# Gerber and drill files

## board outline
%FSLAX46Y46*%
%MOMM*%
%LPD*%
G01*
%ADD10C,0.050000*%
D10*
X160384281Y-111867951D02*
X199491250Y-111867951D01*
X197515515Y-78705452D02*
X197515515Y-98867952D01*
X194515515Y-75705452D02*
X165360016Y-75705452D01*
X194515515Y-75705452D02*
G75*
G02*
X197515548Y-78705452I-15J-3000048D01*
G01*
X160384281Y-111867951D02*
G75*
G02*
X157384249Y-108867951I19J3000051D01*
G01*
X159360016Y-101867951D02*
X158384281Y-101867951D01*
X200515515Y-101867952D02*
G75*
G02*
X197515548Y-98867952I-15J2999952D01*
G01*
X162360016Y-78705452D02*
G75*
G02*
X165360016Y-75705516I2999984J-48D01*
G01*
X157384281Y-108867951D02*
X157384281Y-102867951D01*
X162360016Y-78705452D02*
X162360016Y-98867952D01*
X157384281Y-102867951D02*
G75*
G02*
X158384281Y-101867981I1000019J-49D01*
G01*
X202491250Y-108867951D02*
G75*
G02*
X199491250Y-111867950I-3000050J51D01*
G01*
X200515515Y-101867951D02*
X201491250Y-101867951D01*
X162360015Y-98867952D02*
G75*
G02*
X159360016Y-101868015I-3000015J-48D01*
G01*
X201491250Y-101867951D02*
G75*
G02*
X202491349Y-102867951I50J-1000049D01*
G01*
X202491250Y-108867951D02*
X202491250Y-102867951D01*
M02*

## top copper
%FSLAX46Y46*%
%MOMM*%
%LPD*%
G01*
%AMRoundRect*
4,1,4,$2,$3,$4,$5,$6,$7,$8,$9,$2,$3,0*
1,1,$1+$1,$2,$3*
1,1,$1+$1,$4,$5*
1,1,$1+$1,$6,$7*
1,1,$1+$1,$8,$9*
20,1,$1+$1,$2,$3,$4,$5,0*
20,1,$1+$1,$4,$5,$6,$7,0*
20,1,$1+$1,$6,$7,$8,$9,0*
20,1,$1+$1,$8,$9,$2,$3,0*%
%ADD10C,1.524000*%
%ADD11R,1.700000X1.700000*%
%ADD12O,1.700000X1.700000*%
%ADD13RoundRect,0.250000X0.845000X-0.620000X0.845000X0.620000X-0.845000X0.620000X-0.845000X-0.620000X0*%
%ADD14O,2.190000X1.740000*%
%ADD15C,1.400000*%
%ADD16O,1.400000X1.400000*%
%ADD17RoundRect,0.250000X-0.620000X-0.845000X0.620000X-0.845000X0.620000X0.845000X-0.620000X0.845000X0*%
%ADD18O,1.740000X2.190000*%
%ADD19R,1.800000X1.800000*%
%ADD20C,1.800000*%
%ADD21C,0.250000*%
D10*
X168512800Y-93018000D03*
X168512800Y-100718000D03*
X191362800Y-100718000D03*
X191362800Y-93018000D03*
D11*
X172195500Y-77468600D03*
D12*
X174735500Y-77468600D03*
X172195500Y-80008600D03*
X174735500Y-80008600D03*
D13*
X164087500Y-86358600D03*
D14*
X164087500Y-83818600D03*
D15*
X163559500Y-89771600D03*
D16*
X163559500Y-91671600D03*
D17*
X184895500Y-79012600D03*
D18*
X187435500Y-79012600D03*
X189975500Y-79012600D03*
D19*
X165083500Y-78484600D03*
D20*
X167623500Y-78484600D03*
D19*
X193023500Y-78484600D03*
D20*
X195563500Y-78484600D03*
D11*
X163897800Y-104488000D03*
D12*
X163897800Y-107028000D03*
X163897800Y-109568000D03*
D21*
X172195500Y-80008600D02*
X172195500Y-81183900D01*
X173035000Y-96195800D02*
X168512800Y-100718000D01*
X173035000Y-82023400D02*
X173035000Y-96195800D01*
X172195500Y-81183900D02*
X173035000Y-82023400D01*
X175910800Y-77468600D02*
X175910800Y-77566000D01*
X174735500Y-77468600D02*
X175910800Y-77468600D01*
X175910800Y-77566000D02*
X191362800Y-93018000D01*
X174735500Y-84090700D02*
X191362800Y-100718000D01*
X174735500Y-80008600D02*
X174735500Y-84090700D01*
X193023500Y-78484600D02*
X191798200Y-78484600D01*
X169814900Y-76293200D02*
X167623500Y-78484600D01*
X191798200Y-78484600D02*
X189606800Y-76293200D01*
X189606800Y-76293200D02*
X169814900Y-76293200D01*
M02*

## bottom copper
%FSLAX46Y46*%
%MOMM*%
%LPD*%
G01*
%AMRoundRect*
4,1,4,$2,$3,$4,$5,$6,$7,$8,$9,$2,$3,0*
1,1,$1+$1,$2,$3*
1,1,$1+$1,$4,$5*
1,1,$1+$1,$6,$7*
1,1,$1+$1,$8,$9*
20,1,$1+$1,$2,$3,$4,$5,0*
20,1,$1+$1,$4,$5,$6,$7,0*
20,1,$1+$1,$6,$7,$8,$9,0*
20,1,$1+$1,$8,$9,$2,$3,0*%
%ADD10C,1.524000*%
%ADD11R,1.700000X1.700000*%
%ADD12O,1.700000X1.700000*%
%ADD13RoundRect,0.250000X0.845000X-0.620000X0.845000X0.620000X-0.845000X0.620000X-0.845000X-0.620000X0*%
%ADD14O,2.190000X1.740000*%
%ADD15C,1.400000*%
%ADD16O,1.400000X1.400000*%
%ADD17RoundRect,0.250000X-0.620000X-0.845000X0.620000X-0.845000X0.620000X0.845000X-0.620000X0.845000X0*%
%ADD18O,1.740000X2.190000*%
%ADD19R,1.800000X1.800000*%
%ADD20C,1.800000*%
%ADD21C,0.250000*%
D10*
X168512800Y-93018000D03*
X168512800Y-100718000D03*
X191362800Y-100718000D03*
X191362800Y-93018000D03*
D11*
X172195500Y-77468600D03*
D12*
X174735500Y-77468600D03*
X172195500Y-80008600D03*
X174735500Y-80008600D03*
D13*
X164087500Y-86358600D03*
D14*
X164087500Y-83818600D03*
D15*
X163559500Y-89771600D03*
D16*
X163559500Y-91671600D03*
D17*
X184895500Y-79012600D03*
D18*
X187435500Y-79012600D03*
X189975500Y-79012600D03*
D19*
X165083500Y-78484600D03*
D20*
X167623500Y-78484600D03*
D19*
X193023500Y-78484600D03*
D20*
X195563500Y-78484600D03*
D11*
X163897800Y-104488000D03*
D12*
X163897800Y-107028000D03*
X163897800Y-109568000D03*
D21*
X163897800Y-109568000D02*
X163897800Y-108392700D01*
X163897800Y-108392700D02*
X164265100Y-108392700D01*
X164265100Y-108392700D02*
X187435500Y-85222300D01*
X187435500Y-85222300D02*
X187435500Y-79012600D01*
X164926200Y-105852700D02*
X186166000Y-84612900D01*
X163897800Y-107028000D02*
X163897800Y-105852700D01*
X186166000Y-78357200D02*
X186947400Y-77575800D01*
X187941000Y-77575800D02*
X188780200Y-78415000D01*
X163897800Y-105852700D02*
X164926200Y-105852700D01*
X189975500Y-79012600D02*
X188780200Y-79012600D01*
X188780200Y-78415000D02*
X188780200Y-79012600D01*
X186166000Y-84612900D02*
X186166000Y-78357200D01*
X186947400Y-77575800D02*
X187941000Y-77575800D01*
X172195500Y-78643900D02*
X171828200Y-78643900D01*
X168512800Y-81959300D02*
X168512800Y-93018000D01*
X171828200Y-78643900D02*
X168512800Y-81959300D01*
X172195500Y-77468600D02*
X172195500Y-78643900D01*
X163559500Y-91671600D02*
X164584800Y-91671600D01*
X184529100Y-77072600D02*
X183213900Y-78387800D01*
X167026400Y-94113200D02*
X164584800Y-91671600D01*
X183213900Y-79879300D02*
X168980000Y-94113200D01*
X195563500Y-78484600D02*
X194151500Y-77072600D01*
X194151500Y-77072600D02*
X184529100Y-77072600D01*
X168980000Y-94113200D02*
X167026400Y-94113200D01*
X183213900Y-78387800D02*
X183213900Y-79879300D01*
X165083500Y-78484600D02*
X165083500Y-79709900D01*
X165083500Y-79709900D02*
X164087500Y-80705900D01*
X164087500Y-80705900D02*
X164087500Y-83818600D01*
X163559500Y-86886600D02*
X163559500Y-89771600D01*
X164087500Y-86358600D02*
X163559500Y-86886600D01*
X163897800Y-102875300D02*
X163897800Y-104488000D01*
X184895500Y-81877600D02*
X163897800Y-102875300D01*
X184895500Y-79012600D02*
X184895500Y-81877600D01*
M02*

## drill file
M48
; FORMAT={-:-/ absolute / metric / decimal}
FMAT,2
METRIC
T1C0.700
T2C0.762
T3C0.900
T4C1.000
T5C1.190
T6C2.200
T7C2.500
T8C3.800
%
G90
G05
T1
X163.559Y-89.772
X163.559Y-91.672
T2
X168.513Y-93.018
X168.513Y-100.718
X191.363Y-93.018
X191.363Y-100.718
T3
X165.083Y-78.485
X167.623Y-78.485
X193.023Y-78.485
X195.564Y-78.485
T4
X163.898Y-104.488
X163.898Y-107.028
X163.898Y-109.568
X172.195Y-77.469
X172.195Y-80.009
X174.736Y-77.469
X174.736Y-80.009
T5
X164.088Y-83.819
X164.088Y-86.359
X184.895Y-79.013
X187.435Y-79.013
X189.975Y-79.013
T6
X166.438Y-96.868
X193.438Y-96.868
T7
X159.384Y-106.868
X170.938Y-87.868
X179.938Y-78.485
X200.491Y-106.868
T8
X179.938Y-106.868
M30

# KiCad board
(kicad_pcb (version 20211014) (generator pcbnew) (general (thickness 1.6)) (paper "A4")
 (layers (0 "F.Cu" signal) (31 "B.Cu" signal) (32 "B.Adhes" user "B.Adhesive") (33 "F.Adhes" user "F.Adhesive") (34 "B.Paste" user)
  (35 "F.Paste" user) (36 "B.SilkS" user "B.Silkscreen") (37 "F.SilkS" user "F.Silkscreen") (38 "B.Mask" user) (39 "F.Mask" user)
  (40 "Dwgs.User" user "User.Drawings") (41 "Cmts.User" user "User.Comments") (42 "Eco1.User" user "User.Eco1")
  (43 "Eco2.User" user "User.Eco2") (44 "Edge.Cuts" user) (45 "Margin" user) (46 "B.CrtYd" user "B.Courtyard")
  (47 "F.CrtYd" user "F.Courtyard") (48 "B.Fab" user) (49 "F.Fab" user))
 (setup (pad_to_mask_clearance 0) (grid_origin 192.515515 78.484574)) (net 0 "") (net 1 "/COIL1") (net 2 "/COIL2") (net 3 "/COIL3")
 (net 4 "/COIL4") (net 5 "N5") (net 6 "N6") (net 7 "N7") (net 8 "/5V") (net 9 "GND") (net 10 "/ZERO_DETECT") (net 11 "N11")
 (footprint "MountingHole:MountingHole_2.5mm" (layer "F.Cu") (at 179.9378 78.4846)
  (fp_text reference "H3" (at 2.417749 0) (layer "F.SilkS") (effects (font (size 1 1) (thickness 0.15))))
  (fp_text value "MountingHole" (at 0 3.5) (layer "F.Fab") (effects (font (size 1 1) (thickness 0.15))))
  (pad "" np_thru_hole circle locked (at 0 0) (size 2.5 2.5) (drill 2.5) (layers *.Cu *.Mask)))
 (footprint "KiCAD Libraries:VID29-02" (layer "F.Cu") (at 180.1028 96.868)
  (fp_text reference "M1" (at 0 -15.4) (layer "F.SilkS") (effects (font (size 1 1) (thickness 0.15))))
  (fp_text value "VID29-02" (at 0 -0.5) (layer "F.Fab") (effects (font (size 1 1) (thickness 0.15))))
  (pad "" np_thru_hole circle locked (at -9.165 -9) (size 2.5 2.5) (drill 2.5) (layers *.Cu *.Mask))
  (pad "" np_thru_hole circle locked (at 13.335 0) (size 2.2 2.2) (drill 2.2) (layers *.Cu *.Mask))
  (pad "" np_thru_hole circle locked (at -0.165 10) (size 3.8 3.8) (drill 3.8) (layers *.Cu *.Mask))
  (pad "" np_thru_hole circle locked (at -13.665 0) (size 2.2 2.2) (drill 2.2) (layers *.Cu *.Mask))
  (pad "1" thru_hole circle locked (at -11.59 -3.85) (size 1.524 1.524) (drill 0.762) (layers *.Cu *.Mask) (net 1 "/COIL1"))
  (pad "2" thru_hole circle locked (at -11.59 3.85) (size 1.524 1.524) (drill 0.762) (layers *.Cu *.Mask) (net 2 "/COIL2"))
  (pad "3" thru_hole circle locked (at 11.26 3.85) (size 1.524 1.524) (drill 0.762) (layers *.Cu *.Mask) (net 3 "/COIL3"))
  (pad "4" thru_hole circle locked (at 11.26 -3.85) (size 1.524 1.524) (drill 0.762) (layers *.Cu *.Mask) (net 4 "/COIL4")))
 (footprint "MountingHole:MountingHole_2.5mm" (layer "F.Cu") (at 159.3843 106.868)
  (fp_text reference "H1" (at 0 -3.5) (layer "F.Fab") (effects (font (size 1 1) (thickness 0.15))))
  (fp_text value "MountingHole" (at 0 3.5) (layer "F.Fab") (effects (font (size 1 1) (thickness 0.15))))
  (pad "" np_thru_hole circle locked (at 0 0) (size 2.5 2.5) (drill 2.5) (layers *.Cu *.Mask)))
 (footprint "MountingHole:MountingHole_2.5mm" (layer "F.Cu") (at 200.4913 106.868)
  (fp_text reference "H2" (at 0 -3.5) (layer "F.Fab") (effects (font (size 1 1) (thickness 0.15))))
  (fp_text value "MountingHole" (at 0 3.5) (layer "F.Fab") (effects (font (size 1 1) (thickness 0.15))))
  (pad "" np_thru_hole circle locked (at 0 0) (size 2.5 2.5) (drill 2.5) (layers *.Cu *.Mask)))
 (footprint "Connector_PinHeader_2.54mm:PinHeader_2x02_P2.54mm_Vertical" (layer "F.Cu") (at 172.1955 77.4686)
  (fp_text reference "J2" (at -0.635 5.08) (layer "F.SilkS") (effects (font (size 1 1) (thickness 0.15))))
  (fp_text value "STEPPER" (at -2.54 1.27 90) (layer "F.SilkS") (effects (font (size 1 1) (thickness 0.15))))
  (pad "1" thru_hole rect locked (at 0 0) (size 1.7 1.7) (drill 1) (layers *.Cu *.Mask) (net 1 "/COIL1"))
  (pad "2" thru_hole oval locked (at 2.54 0) (size 1.7 1.7) (drill 1) (layers *.Cu *.Mask) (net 4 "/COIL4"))
  (pad "3" thru_hole oval locked (at 0 2.54) (size 1.7 1.7) (drill 1) (layers *.Cu *.Mask) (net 2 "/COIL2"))
  (pad "4" thru_hole oval locked (at 2.54 2.54) (size 1.7 1.7) (drill 1) (layers *.Cu *.Mask) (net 3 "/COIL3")))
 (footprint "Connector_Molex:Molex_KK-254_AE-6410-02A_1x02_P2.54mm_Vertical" (layer "F.Cu") (at 164.0875 86.3586 90)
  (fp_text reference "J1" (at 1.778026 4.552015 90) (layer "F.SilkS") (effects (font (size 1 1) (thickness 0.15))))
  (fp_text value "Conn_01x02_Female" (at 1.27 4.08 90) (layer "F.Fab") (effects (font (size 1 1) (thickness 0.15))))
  (pad "1" thru_hole roundrect (at 0 0 90) (size 1.74 2.19) (drill 1.19) (layers *.Cu *.Mask) (roundrect_rratio 0.143678) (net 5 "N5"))
  (pad "2" thru_hole oval (at 2.54 0 90) (size 1.74 2.19) (drill 1.19) (layers *.Cu *.Mask) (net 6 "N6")))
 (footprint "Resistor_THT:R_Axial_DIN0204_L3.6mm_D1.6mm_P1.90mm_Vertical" (layer "F.Cu") (at 163.5595 89.7716 -90)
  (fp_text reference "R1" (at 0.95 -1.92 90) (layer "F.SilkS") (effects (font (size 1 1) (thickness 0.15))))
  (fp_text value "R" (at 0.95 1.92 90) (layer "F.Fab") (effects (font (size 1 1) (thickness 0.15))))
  (pad "1" thru_hole circle (at 0 0 270) (size 1.4 1.4) (drill 0.7) (layers *.Cu *.Mask) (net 5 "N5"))
  (pad "2" thru_hole oval (at 1.9 0 270) (size 1.4 1.4) (drill 0.7) (layers *.Cu *.Mask) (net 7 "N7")))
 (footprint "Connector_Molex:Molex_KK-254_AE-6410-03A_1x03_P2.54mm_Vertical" (layer "F.Cu") (at 184.8955 79.0126)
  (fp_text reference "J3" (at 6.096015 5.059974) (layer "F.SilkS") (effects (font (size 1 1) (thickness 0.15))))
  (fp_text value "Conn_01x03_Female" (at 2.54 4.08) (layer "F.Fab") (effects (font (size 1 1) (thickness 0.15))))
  (pad "1" thru_hole roundrect (at 0 0) (size 1.74 2.19) (drill 1.19) (layers *.Cu *.Mask) (roundrect_rratio 0.143678) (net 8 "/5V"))
  (pad "2" thru_hole oval (at 2.54 0) (size 1.74 2.19) (drill 1.19) (layers *.Cu *.Mask) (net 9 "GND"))
  (pad "3" thru_hole oval (at 5.08 0) (size 1.74 2.19) (drill 1.19) (layers *.Cu *.Mask) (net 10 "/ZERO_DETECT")))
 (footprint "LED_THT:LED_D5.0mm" (layer "F.Cu") (at 165.0835 78.4846)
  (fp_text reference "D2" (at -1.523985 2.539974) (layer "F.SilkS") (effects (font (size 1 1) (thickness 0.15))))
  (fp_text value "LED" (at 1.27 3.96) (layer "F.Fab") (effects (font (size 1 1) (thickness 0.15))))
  (pad "1" thru_hole rect (at 0 0) (size 1.8 1.8) (drill 0.9) (layers *.Cu *.Mask) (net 6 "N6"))
  (pad "2" thru_hole circle (at 2.54 0) (size 1.8 1.8) (drill 0.9) (layers *.Cu *.Mask) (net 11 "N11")))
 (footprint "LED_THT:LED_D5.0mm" (layer "F.Cu") (at 193.0235 78.4846)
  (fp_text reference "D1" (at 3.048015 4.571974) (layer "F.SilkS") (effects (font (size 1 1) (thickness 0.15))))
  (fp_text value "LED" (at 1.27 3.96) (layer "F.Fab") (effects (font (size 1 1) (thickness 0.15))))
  (pad "1" thru_hole rect (at 0 0) (size 1.8 1.8) (drill 0.9) (layers *.Cu *.Mask) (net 11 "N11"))
  (pad "2" thru_hole circle (at 2.54 0) (size 1.8 1.8) (drill 0.9) (layers *.Cu *.Mask) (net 7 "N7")))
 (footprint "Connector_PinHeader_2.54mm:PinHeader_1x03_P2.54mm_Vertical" (layer "B.Cu") (at 163.8978 104.488 180)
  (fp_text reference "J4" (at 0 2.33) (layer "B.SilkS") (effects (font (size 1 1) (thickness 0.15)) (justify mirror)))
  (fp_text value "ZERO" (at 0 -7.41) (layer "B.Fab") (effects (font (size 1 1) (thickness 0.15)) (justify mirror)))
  (pad "1" thru_hole rect locked (at 0 0 180) (size 1.7 1.7) (drill 1) (layers *.Cu *.Mask) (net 8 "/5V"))
  (pad "2" thru_hole oval locked (at 0 -2.54 180) (size 1.7 1.7) (drill 1) (layers *.Cu *.Mask) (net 10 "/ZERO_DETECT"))
  (pad "3" thru_hole oval locked (at 0 -5.08 180) (size 1.7 1.7) (drill 1) (layers *.Cu *.Mask) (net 9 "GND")))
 (gr_line (start 160.384281 111.867951) (end 199.49125 111.867951) (layer "Edge.Cuts") (width 0.05))
 (gr_line (start 197.515515 78.705452) (end 197.515515 98.867952) (layer "Edge.Cuts") (width 0.05))
 (gr_line (start 194.515515 75.705452) (end 165.360016 75.705452) (layer "Edge.Cuts") (width 0.05))
 (gr_arc (start 194.515515 75.705452) (mid 196.636835 76.584132) (end 197.515515 78.705452) (layer "Edge.Cuts") (width 0.05))
 (gr_arc (start 160.384281 111.867951) (mid 158.262961 110.989271) (end 157.384281 108.867951) (layer "Edge.Cuts") (width 0.05))
 (gr_line (start 159.360016 101.867951) (end 158.384281 101.867951) (layer "Edge.Cuts") (width 0.05))
 (gr_arc (start 200.515515 101.867952) (mid 198.394195 100.989272) (end 197.515515 98.867952) (layer "Edge.Cuts") (width 0.05))
 (gr_arc (start 162.360016 78.705452) (mid 163.238696 76.584132) (end 165.360016 75.705452) (layer "Edge.Cuts") (width 0.05))
 (gr_line (start 157.384281 108.867951) (end 157.384281 102.867951) (layer "Edge.Cuts") (width 0.05))
 (gr_line (start 162.360016 78.705452) (end 162.360016 98.867952) (layer "Edge.Cuts") (width 0.05))
 (gr_arc (start 157.384281 102.867951) (mid 157.677174 102.160844) (end 158.384281 101.867951) (layer "Edge.Cuts") (width 0.05))
 (gr_arc (start 202.49125 108.867951) (mid 201.61257 110.989271) (end 199.49125 111.867951) (layer "Edge.Cuts") (width 0.05))
 (gr_line (start 200.515515 101.867951) (end 201.49125 101.867951) (layer "Edge.Cuts") (width 0.05))
 (gr_arc (start 162.360015 98.867952) (mid 161.481336 100.989272) (end 159.360016 101.867951) (layer "Edge.Cuts") (width 0.05))
 (gr_arc (start 201.49125 101.867951) (mid 202.198357 102.160844) (end 202.49125 102.867951) (layer "Edge.Cuts") (width 0.05))
 (gr_line (start 202.49125 108.867951) (end 202.49125 102.867951) (layer "Edge.Cuts") (width 0.05))
 (segment (start 163.8978 109.568) (end 163.8978 108.3927) (width 0.25) (layer "B.Cu") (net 9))
 (segment (start 163.8978 108.3927) (end 164.2651 108.3927) (width 0.25) (layer "B.Cu") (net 9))
 (segment (start 164.2651 108.3927) (end 187.4355 85.2223) (width 0.25) (layer "B.Cu") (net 9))
 (segment (start 187.4355 85.2223) (end 187.4355 79.0126) (width 0.25) (layer "B.Cu") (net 9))
 (segment (start 164.9262 105.8527) (end 186.166 84.6129) (width 0.25) (layer "B.Cu") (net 10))
 (segment (start 163.8978 107.028) (end 163.8978 105.8527) (width 0.25) (layer "B.Cu") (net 10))
 (segment (start 186.166 78.3572) (end 186.9474 77.5758) (width 0.25) (layer "B.Cu") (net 10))
 (segment (start 187.941 77.5758) (end 188.7802 78.415) (width 0.25) (layer "B.Cu") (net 10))
 (segment (start 163.8978 105.8527) (end 164.9262 105.8527) (width 0.25) (layer "B.Cu") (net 10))
 (segment (start 189.9755 79.0126) (end 188.7802 79.0126) (width 0.25) (layer "B.Cu") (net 10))
 (segment (start 188.7802 78.415) (end 188.7802 79.0126) (width 0.25) (layer "B.Cu") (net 10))
 (segment (start 186.166 84.6129) (end 186.166 78.3572) (width 0.25) (layer "B.Cu") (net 10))
 (segment (start 186.9474 77.5758) (end 187.941 77.5758) (width 0.25) (layer "B.Cu") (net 10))
 (segment (start 172.1955 80.0086) (end 172.1955 81.1839) (width 0.25) (layer "F.Cu") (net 2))
 (segment (start 173.035 96.1958) (end 168.5128 100.718) (width 0.25) (layer "F.Cu") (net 2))
 (segment (start 173.035 82.0234) (end 173.035 96.1958) (width 0.25) (layer "F.Cu") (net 2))
 (segment (start 172.1955 81.1839) (end 173.035 82.0234) (width 0.25) (layer "F.Cu") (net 2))
 (segment (start 172.1955 78.6439) (end 171.8282 78.6439) (width 0.25) (layer "B.Cu") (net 1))
 (segment (start 168.5128 81.9593) (end 168.5128 93.018) (width 0.25) (layer "B.Cu") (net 1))
 (segment (start 171.8282 78.6439) (end 168.5128 81.9593) (width 0.25) (layer "B.Cu") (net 1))
 (segment (start 172.1955 77.4686) (end 172.1955 78.6439) (width 0.25) (layer "B.Cu") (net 1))
 (segment (start 175.9108 77.4686) (end 175.9108 77.566) (width 0.25) (layer "F.Cu") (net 4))
 (segment (start 174.7355 77.4686) (end 175.9108 77.4686) (width 0.25) (layer "F.Cu") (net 4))
 (segment (start 175.9108 77.566) (end 191.3628 93.018) (width 0.25) (layer "F.Cu") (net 4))
 (segment (start 174.7355 84.0907) (end 191.3628 100.718) (width 0.25) (layer "F.Cu") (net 3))
 (segment (start 174.7355 80.0086) (end 174.7355 84.0907) (width 0.25) (layer "F.Cu") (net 3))
 (segment (start 193.0235 78.4846) (end 191.7982 78.4846) (width 0.25) (layer "F.Cu") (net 11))
 (segment (start 169.8149 76.2932) (end 167.6235 78.4846) (width 0.25) (layer "F.Cu") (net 11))
 (segment (start 191.7982 78.4846) (end 189.6068 76.2932) (width 0.25) (layer "F.Cu") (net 11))
 (segment (start 189.6068 76.2932) (end 169.8149 76.2932) (width 0.25) (layer "F.Cu") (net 11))
 (segment (start 163.5595 91.6716) (end 164.5848 91.6716) (width 0.25) (layer "B.Cu") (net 7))
 (segment (start 184.5291 77.0726) (end 183.2139 78.3878) (width 0.25) (layer "B.Cu") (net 7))
 (segment (start 167.0264 94.1132) (end 164.5848 91.6716) (width 0.25) (layer "B.Cu") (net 7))
 (segment (start 183.2139 79.8793) (end 168.98 94.1132) (width 0.25) (layer "B.Cu") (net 7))
 (segment (start 195.5635 78.4846) (end 194.1515 77.0726) (width 0.25) (layer "B.Cu") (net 7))
 (segment (start 194.1515 77.0726) (end 184.5291 77.0726) (width 0.25) (layer "B.Cu") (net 7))
 (segment (start 168.98 94.1132) (end 167.0264 94.1132) (width 0.25) (layer "B.Cu") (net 7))
 (segment (start 183.2139 78.3878) (end 183.2139 79.8793) (width 0.25) (layer "B.Cu") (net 7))
 (segment (start 165.0835 78.4846) (end 165.0835 79.7099) (width 0.25) (layer "B.Cu") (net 6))
 (segment (start 165.0835 79.7099) (end 164.0875 80.7059) (width 0.25) (layer "B.Cu") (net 6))
 (segment (start 164.0875 80.7059) (end 164.0875 83.8186) (width 0.25) (layer "B.Cu") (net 6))
 (segment (start 163.5595 86.8866) (end 163.5595 89.7716) (width 0.25) (layer "B.Cu") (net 5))
 (segment (start 164.0875 86.3586) (end 163.5595 86.8866) (width 0.25) (layer "B.Cu") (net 5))
 (segment (start 163.8978 102.8753) (end 163.8978 104.488) (width 0.25) (layer "B.Cu") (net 8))
 (segment (start 184.8955 81.8776) (end 163.8978 102.8753) (width 0.25) (layer "B.Cu") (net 8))
 (segment (start 184.8955 79.0126) (end 184.8955 81.8776) (width 0.25) (layer "B.Cu") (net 8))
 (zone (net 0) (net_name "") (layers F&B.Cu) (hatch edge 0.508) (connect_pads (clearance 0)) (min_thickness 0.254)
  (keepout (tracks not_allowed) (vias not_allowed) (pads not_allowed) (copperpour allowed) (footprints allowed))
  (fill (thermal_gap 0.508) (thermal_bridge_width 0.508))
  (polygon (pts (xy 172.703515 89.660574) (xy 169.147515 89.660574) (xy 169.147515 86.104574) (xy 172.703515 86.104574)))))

